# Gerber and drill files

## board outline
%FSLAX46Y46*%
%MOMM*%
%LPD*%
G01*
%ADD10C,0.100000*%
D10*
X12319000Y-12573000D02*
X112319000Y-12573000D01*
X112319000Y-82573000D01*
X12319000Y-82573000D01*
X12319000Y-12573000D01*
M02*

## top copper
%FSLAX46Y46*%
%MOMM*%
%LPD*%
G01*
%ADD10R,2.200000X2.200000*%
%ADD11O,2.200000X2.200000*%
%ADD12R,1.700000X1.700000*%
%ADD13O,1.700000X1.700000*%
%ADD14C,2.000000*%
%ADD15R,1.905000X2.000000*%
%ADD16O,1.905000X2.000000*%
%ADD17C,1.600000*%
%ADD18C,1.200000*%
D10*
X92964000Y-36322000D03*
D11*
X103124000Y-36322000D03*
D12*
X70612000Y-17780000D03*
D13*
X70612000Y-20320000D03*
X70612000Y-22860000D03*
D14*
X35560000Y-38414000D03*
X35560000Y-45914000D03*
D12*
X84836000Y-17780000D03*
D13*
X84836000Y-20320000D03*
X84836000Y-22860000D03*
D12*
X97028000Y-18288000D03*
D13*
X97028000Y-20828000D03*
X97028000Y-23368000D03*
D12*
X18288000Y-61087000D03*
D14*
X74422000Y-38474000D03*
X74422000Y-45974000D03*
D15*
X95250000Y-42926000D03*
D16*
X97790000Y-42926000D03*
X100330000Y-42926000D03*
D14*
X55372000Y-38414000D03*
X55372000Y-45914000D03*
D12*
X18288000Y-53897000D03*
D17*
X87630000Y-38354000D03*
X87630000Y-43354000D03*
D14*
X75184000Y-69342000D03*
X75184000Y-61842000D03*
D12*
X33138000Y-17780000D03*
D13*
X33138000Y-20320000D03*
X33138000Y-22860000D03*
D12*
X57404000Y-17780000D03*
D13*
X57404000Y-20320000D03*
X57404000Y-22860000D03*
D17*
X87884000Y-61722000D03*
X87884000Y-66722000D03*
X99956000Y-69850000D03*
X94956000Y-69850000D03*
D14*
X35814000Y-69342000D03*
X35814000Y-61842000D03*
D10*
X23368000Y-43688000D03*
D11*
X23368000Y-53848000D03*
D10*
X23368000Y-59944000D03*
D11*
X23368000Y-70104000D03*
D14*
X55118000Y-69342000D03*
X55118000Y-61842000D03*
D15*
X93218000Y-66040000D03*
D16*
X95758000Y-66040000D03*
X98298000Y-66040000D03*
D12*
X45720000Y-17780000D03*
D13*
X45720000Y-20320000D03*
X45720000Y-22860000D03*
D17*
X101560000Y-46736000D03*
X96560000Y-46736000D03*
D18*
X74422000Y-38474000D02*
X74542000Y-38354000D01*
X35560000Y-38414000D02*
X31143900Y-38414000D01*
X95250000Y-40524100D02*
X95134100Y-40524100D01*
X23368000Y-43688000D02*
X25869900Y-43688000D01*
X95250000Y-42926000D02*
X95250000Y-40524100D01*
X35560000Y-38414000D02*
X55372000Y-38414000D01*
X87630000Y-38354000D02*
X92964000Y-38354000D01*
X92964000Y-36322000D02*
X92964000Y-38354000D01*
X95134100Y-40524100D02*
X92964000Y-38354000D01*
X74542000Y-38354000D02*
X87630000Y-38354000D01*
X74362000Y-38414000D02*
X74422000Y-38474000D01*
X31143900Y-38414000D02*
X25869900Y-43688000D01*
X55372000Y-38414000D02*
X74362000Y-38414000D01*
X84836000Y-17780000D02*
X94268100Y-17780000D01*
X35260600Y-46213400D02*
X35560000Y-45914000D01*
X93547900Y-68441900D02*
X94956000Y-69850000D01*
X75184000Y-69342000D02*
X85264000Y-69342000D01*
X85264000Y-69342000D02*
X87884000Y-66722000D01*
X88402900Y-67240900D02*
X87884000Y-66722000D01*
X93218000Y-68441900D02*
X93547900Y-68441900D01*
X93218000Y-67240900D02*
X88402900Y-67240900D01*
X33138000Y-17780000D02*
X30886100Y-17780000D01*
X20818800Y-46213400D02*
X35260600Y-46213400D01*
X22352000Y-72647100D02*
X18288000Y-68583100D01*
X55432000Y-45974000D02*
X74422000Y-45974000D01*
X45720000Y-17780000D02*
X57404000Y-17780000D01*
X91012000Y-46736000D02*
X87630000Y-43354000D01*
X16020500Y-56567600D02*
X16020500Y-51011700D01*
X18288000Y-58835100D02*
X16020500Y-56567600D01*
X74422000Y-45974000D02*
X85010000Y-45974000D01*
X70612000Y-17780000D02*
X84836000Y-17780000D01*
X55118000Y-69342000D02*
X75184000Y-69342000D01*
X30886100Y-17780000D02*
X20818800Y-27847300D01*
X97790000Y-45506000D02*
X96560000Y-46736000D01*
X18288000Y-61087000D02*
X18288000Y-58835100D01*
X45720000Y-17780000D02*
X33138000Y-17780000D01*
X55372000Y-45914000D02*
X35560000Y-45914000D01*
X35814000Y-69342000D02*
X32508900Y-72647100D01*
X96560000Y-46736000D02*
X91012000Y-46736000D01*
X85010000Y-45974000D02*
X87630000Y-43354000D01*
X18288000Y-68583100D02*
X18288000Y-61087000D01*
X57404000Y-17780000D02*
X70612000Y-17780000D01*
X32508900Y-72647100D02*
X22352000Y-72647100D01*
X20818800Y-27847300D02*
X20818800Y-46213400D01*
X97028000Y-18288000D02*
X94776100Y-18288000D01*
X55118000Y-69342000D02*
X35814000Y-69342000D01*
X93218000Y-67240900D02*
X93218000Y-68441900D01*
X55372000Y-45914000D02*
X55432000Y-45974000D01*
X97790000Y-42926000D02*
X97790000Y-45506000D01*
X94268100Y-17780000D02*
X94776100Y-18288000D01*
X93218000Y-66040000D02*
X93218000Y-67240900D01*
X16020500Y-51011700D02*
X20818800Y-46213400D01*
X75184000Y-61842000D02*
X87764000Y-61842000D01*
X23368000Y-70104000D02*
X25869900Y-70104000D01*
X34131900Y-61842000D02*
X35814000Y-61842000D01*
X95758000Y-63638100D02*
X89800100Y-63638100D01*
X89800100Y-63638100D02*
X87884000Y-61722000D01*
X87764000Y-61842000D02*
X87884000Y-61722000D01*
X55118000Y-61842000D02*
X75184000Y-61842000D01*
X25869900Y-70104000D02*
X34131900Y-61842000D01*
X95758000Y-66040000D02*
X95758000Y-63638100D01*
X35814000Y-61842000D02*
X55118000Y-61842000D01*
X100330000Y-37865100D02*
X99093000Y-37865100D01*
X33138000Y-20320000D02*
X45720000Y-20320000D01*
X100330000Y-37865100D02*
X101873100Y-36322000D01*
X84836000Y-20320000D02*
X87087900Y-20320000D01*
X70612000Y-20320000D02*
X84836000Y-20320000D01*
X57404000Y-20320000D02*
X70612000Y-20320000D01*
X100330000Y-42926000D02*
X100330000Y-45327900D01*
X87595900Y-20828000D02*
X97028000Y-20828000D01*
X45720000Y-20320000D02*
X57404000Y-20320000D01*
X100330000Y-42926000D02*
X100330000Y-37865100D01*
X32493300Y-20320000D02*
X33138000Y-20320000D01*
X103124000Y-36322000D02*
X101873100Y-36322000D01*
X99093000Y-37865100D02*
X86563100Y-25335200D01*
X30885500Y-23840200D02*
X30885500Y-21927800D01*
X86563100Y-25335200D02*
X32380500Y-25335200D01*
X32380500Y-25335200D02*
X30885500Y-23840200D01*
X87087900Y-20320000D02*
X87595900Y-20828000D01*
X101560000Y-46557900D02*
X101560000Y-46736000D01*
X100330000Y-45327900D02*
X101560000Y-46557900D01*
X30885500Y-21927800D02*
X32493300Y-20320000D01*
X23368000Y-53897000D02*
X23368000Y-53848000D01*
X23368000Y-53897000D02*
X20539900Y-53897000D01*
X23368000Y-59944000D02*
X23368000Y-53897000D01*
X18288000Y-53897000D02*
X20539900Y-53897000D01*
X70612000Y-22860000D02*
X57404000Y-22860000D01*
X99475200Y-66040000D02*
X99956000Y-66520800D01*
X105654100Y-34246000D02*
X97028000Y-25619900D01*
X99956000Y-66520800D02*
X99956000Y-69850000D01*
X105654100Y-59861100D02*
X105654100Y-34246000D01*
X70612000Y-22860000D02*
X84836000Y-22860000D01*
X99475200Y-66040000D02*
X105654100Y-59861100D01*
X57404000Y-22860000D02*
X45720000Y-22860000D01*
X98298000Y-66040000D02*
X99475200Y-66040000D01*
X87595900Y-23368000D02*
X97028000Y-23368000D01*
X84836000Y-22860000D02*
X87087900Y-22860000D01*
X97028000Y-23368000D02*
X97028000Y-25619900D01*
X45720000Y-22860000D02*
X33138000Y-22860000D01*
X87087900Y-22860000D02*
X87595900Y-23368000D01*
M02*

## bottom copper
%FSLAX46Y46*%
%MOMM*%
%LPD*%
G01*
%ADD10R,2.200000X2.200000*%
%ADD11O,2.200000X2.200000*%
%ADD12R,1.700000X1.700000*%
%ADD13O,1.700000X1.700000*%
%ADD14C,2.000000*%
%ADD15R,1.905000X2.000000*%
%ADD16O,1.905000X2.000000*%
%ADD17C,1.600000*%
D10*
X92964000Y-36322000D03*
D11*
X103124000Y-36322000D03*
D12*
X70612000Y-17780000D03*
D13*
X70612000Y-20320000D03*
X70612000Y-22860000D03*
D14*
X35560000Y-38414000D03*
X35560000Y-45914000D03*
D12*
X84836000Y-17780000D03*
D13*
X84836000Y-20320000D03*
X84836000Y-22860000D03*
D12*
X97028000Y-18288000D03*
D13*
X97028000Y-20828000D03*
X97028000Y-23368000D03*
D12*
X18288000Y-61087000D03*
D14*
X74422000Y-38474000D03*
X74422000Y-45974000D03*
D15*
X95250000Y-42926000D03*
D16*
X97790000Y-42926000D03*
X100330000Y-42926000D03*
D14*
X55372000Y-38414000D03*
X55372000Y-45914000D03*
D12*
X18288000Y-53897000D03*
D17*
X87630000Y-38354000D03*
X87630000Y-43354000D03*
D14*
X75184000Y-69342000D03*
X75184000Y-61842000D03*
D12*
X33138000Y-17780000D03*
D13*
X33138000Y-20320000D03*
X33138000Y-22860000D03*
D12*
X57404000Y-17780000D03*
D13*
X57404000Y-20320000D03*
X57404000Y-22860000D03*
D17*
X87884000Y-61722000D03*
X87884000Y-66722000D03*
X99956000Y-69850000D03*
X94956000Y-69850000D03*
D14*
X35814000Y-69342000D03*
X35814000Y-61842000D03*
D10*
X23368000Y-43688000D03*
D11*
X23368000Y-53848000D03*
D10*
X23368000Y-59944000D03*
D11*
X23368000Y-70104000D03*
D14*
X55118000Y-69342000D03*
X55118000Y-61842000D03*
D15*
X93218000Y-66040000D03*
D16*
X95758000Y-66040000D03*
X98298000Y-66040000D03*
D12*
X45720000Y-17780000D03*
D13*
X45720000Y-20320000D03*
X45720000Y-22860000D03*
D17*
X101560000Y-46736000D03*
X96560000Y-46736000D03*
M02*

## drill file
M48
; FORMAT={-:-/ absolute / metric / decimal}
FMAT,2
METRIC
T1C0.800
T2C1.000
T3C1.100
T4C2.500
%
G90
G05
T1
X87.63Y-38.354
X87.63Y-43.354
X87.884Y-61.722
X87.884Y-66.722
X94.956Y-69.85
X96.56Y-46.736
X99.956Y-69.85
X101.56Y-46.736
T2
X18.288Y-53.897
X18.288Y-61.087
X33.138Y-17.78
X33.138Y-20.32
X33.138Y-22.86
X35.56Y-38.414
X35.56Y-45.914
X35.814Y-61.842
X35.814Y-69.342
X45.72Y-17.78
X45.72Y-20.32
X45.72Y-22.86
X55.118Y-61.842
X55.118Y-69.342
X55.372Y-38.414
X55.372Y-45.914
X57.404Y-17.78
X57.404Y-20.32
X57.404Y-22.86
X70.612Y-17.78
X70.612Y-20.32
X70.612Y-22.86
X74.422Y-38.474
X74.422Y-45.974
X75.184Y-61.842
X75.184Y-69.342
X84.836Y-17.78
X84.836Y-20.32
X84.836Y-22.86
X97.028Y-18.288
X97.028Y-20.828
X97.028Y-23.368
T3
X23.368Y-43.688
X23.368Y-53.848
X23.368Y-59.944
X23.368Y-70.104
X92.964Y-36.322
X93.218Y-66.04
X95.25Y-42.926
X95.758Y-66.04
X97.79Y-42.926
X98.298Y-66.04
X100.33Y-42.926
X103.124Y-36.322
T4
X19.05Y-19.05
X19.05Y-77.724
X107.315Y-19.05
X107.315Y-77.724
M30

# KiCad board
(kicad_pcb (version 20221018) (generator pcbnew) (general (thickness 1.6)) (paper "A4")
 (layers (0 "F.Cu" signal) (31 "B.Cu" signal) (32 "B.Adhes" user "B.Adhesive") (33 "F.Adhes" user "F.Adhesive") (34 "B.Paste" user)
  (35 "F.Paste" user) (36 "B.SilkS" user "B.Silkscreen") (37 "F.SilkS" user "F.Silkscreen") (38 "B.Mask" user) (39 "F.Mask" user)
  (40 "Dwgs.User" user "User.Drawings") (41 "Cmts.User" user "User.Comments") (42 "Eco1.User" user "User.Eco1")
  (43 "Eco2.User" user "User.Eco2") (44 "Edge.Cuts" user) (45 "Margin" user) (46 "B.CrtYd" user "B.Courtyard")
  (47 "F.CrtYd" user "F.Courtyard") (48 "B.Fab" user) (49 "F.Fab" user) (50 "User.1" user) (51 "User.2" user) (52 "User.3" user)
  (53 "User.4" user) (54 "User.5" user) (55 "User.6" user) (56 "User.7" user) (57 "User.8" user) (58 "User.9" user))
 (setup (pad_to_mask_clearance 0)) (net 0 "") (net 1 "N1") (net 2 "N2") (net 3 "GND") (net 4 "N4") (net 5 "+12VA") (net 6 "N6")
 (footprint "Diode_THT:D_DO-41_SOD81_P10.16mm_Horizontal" (layer "F.Cu") (at 92.964 36.322)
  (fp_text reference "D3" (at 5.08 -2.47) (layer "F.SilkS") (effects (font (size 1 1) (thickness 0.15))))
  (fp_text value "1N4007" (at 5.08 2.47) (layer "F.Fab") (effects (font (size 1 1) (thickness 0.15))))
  (pad "1" thru_hole rect (at 0 0) (size 2.2 2.2) (drill 1.1) (layers "*.Cu" "*.Mask") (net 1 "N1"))
  (pad "2" thru_hole oval (at 10.16 0) (size 2.2 2.2) (drill 1.1) (layers "*.Cu" "*.Mask") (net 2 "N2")))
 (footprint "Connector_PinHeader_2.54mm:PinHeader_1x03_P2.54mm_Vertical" (layer "F.Cu") (at 70.612 17.78)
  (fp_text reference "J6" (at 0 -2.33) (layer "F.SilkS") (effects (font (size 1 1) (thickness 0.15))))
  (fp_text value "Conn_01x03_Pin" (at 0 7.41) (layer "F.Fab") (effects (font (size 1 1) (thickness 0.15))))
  (pad "1" thru_hole rect (at 0 0) (size 1.7 1.7) (drill 1) (layers "*.Cu" "*.Mask") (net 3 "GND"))
  (pad "2" thru_hole oval (at 0 2.54) (size 1.7 1.7) (drill 1) (layers "*.Cu" "*.Mask") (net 2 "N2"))
  (pad "3" thru_hole oval (at 0 5.08) (size 1.7 1.7) (drill 1) (layers "*.Cu" "*.Mask") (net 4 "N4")))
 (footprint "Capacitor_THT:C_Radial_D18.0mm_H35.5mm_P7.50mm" (layer "F.Cu") (at 35.56 38.414 -90)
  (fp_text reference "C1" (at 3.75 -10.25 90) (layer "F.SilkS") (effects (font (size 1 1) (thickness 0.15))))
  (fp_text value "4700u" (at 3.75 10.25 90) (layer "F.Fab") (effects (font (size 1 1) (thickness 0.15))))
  (pad "1" thru_hole circle (at 0 0 270) (size 2 2) (drill 1) (layers "*.Cu" "*.Mask") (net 1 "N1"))
  (pad "2" thru_hole circle (at 7.5 0 270) (size 2 2) (drill 1) (layers "*.Cu" "*.Mask") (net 3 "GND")))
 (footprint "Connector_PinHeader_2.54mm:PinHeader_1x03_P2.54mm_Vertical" (layer "F.Cu") (at 84.836 17.78)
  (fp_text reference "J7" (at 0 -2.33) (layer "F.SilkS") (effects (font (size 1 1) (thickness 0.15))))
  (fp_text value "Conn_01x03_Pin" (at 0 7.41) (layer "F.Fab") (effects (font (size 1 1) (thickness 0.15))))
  (pad "1" thru_hole rect (at 0 0) (size 1.7 1.7) (drill 1) (layers "*.Cu" "*.Mask") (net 3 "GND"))
  (pad "2" thru_hole oval (at 0 2.54) (size 1.7 1.7) (drill 1) (layers "*.Cu" "*.Mask") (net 2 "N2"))
  (pad "3" thru_hole oval (at 0 5.08) (size 1.7 1.7) (drill 1) (layers "*.Cu" "*.Mask") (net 4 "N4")))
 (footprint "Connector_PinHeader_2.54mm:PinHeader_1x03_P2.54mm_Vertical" (layer "F.Cu") (at 97.028 18.288)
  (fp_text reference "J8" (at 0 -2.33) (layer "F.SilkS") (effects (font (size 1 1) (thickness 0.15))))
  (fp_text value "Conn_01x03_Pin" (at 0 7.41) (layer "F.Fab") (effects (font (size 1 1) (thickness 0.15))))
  (pad "1" thru_hole rect (at 0 0) (size 1.7 1.7) (drill 1) (layers "*.Cu" "*.Mask") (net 3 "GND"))
  (pad "2" thru_hole oval (at 0 2.54) (size 1.7 1.7) (drill 1) (layers "*.Cu" "*.Mask") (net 2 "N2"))
  (pad "3" thru_hole oval (at 0 5.08) (size 1.7 1.7) (drill 1) (layers "*.Cu" "*.Mask") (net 4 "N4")))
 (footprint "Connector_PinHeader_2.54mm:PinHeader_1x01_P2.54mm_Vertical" (layer "F.Cu") (at 18.288 61.087)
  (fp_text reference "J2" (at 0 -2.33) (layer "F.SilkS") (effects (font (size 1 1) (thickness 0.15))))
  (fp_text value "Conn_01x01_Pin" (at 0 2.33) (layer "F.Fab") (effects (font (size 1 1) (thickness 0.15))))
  (pad "1" thru_hole rect (at 0 0) (size 1.7 1.7) (drill 1) (layers "*.Cu" "*.Mask") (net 3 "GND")))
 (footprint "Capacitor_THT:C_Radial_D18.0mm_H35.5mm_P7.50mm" (layer "F.Cu") (at 74.422 38.474 -90)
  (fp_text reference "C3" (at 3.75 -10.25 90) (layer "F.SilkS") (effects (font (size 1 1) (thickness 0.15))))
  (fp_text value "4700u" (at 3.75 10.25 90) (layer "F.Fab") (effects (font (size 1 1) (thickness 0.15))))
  (pad "1" thru_hole circle (at 0 0 270) (size 2 2) (drill 1) (layers "*.Cu" "*.Mask") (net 1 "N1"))
  (pad "2" thru_hole circle (at 7.5 0 270) (size 2 2) (drill 1) (layers "*.Cu" "*.Mask") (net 3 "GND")))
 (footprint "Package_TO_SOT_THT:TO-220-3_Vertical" (layer "F.Cu") (at 95.25 42.926)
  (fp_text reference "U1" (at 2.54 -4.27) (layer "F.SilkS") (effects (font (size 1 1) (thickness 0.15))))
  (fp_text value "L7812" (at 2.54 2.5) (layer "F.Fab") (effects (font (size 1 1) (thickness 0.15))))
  (pad "1" thru_hole rect (at 0 0) (size 1.905 2) (drill 1.1) (layers "*.Cu" "*.Mask") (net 1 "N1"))
  (pad "2" thru_hole oval (at 2.54 0) (size 1.905 2) (drill 1.1) (layers "*.Cu" "*.Mask") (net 3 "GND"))
  (pad "3" thru_hole oval (at 5.08 0) (size 1.905 2) (drill 1.1) (layers "*.Cu" "*.Mask") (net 2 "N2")))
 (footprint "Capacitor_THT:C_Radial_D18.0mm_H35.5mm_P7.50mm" (layer "F.Cu") (at 55.372 38.414 -90)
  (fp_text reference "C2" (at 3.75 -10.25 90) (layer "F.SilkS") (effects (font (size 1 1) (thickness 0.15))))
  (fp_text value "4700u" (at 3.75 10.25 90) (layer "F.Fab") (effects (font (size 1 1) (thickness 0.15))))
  (pad "1" thru_hole circle (at 0 0 270) (size 2 2) (drill 1) (layers "*.Cu" "*.Mask") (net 1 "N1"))
  (pad "2" thru_hole circle (at 7.5 0 270) (size 2 2) (drill 1) (layers "*.Cu" "*.Mask") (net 3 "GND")))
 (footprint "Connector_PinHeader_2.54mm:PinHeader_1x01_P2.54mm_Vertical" (layer "F.Cu") (at 18.288 53.897)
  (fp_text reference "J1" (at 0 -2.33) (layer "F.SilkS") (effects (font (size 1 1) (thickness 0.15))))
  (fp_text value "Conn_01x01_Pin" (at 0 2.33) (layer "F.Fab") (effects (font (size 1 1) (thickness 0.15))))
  (pad "1" thru_hole rect (at 0 0) (size 1.7 1.7) (drill 1) (layers "*.Cu" "*.Mask") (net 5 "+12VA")))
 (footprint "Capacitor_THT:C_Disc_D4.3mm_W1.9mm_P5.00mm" (layer "F.Cu") (at 87.63 38.354 -90)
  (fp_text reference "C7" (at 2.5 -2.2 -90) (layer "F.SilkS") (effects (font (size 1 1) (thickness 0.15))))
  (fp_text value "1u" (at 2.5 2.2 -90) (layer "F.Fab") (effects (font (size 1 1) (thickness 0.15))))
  (pad "1" thru_hole circle (at 0 0 270) (size 1.6 1.6) (drill 0.8) (layers "*.Cu" "*.Mask") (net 1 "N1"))
  (pad "2" thru_hole circle (at 5 0 270) (size 1.6 1.6) (drill 0.8) (layers "*.Cu" "*.Mask") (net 3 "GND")))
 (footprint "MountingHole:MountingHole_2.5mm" (layer "F.Cu") (at 19.05 19.05)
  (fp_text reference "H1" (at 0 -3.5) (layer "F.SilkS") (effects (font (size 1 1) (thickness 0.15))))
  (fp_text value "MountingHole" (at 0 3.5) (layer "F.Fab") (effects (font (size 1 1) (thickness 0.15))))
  (pad "" np_thru_hole circle (at 0 0) (size 2.5 2.5) (drill 2.5) (layers "*.Cu" "*.Mask")))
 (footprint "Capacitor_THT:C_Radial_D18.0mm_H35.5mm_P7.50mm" (layer "F.Cu") (at 75.184 69.342 90)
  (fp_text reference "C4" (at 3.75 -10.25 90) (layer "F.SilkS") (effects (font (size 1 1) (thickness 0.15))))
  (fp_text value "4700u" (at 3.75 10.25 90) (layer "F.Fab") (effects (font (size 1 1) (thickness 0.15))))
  (pad "1" thru_hole circle (at 0 0 90) (size 2 2) (drill 1) (layers "*.Cu" "*.Mask") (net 3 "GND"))
  (pad "2" thru_hole circle (at 7.5 0 90) (size 2 2) (drill 1) (layers "*.Cu" "*.Mask") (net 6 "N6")))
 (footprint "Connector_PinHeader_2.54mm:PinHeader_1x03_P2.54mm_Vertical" (layer "F.Cu") (at 33.138 17.78)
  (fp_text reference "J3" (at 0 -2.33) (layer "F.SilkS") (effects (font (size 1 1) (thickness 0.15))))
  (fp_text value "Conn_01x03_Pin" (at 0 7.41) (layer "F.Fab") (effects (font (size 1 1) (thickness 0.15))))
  (pad "1" thru_hole rect (at 0 0) (size 1.7 1.7) (drill 1) (layers "*.Cu" "*.Mask") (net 3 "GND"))
  (pad "2" thru_hole oval (at 0 2.54) (size 1.7 1.7) (drill 1) (layers "*.Cu" "*.Mask") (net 2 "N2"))
  (pad "3" thru_hole oval (at 0 5.08) (size 1.7 1.7) (drill 1) (layers "*.Cu" "*.Mask") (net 4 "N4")))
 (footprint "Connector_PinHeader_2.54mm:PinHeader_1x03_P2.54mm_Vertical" (layer "F.Cu") (at 57.404 17.78)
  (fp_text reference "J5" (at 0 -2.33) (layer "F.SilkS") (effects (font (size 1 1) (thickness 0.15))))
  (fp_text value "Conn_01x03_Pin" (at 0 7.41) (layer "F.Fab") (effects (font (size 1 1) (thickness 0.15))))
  (pad "1" thru_hole rect (at 0 0) (size 1.7 1.7) (drill 1) (layers "*.Cu" "*.Mask") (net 3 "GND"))
  (pad "2" thru_hole oval (at 0 2.54) (size 1.7 1.7) (drill 1) (layers "*.Cu" "*.Mask") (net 2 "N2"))
  (pad "3" thru_hole oval (at 0 5.08) (size 1.7 1.7) (drill 1) (layers "*.Cu" "*.Mask") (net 4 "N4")))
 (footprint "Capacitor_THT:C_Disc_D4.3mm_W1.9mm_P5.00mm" (layer "F.Cu") (at 87.884 61.722 -90)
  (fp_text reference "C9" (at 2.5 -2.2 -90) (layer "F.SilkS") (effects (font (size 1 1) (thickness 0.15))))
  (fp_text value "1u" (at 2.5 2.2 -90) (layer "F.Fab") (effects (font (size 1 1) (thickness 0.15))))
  (pad "1" thru_hole circle (at 0 0 270) (size 1.6 1.6) (drill 0.8) (layers "*.Cu" "*.Mask") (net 6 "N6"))
  (pad "2" thru_hole circle (at 5 0 270) (size 1.6 1.6) (drill 0.8) (layers "*.Cu" "*.Mask") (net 3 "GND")))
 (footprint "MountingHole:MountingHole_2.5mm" (layer "F.Cu") (at 19.05 77.724)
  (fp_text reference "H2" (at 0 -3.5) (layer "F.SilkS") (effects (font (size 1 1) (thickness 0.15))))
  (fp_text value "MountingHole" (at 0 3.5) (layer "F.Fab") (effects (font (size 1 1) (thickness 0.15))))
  (pad "" np_thru_hole circle (at 0 0) (size 2.5 2.5) (drill 2.5) (layers "*.Cu" "*.Mask")))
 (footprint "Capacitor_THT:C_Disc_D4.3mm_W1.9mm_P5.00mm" (layer "F.Cu") (at 99.956 69.85 180)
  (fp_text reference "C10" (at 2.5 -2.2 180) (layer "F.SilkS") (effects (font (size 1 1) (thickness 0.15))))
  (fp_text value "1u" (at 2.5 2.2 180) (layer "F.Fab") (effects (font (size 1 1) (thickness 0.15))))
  (pad "1" thru_hole circle (at 0 0 180) (size 1.6 1.6) (drill 0.8) (layers "*.Cu" "*.Mask") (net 4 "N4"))
  (pad "2" thru_hole circle (at 5 0 180) (size 1.6 1.6) (drill 0.8) (layers "*.Cu" "*.Mask") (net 3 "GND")))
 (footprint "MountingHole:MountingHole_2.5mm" (layer "F.Cu") (at 107.315 77.724)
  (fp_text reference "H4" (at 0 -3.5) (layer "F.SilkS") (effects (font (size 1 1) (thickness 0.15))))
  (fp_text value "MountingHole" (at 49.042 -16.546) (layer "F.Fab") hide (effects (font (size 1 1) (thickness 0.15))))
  (pad "" np_thru_hole circle (at 0 0) (size 2.5 2.5) (drill 2.5) (layers "*.Cu" "*.Mask")))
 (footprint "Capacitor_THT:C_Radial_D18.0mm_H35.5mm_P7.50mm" (layer "F.Cu") (at 35.814 69.342 90)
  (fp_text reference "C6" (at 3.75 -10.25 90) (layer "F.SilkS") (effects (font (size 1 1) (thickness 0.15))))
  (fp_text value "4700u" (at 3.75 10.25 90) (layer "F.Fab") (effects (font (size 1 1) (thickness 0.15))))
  (pad "1" thru_hole circle (at 0 0 90) (size 2 2) (drill 1) (layers "*.Cu" "*.Mask") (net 3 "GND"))
  (pad "2" thru_hole circle (at 7.5 0 90) (size 2 2) (drill 1) (layers "*.Cu" "*.Mask") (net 6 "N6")))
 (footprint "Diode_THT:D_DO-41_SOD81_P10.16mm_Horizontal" (layer "F.Cu") (at 23.368 43.688 -90)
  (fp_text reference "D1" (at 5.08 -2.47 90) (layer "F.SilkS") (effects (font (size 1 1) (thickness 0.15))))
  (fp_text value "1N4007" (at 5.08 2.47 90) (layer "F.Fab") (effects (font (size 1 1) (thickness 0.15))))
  (pad "1" thru_hole rect (at 0 0 270) (size 2.2 2.2) (drill 1.1) (layers "*.Cu" "*.Mask") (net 1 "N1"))
  (pad "2" thru_hole oval (at 10.16 0 270) (size 2.2 2.2) (drill 1.1) (layers "*.Cu" "*.Mask") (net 5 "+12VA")))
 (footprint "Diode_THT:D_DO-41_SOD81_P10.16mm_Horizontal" (layer "F.Cu") (at 23.368 59.944 -90)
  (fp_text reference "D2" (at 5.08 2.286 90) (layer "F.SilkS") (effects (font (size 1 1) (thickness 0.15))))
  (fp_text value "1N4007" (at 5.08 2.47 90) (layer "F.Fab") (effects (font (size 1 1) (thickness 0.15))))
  (pad "1" thru_hole rect (at 0 0 270) (size 2.2 2.2) (drill 1.1) (layers "*.Cu" "*.Mask") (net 5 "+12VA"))
  (pad "2" thru_hole oval (at 10.16 0 270) (size 2.2 2.2) (drill 1.1) (layers "*.Cu" "*.Mask") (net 6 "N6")))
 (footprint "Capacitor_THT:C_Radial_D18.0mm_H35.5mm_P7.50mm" (layer "F.Cu") (at 55.118 69.342 90)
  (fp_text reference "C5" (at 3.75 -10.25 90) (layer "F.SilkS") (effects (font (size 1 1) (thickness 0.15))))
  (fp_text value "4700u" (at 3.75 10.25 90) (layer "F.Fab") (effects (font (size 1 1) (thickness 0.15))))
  (pad "1" thru_hole circle (at 0 0 90) (size 2 2) (drill 1) (layers "*.Cu" "*.Mask") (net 3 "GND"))
  (pad "2" thru_hole circle (at 7.5 0 90) (size 2 2) (drill 1) (layers "*.Cu" "*.Mask") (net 6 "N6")))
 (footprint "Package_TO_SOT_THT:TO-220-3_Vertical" (layer "F.Cu") (at 93.218 66.04)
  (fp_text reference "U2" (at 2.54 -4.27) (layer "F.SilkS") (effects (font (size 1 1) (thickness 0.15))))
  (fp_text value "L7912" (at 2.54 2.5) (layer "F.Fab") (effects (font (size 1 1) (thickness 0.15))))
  (pad "1" thru_hole rect (at 0 0) (size 1.905 2) (drill 1.1) (layers "*.Cu" "*.Mask") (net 3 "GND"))
  (pad "2" thru_hole oval (at 2.54 0) (size 1.905 2) (drill 1.1) (layers "*.Cu" "*.Mask") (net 6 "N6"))
  (pad "3" thru_hole oval (at 5.08 0) (size 1.905 2) (drill 1.1) (layers "*.Cu" "*.Mask") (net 4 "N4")))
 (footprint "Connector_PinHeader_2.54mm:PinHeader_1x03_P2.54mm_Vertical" (layer "F.Cu") (at 45.72 17.78)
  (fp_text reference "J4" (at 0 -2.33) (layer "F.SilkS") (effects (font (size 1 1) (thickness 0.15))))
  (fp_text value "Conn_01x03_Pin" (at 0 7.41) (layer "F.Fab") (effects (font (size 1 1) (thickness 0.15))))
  (pad "1" thru_hole rect (at 0 0) (size 1.7 1.7) (drill 1) (layers "*.Cu" "*.Mask") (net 3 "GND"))
  (pad "2" thru_hole oval (at 0 2.54) (size 1.7 1.7) (drill 1) (layers "*.Cu" "*.Mask") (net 2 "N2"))
  (pad "3" thru_hole oval (at 0 5.08) (size 1.7 1.7) (drill 1) (layers "*.Cu" "*.Mask") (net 4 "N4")))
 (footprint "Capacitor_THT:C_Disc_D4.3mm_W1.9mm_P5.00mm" (layer "F.Cu") (at 101.56 46.736 180)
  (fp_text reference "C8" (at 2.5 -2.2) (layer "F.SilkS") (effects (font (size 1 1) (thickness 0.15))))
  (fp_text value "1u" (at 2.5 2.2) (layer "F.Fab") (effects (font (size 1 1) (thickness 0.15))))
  (pad "1" thru_hole circle (at 0 0 180) (size 1.6 1.6) (drill 0.8) (layers "*.Cu" "*.Mask") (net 2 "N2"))
  (pad "2" thru_hole circle (at 5 0 180) (size 1.6 1.6) (drill 0.8) (layers "*.Cu" "*.Mask") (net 3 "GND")))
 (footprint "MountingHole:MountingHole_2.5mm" (layer "F.Cu") (at 107.315 19.05)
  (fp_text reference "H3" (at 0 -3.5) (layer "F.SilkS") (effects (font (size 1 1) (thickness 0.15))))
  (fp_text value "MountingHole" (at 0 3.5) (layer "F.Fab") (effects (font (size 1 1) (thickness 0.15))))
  (pad "" np_thru_hole circle (at 0 0) (size 2.5 2.5) (drill 2.5) (layers "*.Cu" "*.Mask")))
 (gr_rect (start 12.319 12.573) (end 112.319 82.573) (stroke (width 0.1) (type default)) (fill none) (layer "Edge.Cuts"))
 (segment (start 74.422 38.474) (end 74.542 38.354) (width 1.2) (layer "F.Cu") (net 1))
 (segment (start 35.56 38.414) (end 31.1439 38.414) (width 1.2) (layer "F.Cu") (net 1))
 (segment (start 95.25 40.5241) (end 95.1341 40.5241) (width 1.2) (layer "F.Cu") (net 1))
 (segment (start 23.368 43.688) (end 25.8699 43.688) (width 1.2) (layer "F.Cu") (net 1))
 (segment (start 95.25 42.926) (end 95.25 40.5241) (width 1.2) (layer "F.Cu") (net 1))
 (segment (start 35.56 38.414) (end 55.372 38.414) (width 1.2) (layer "F.Cu") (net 1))
 (segment (start 87.63 38.354) (end 92.964 38.354) (width 1.2) (layer "F.Cu") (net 1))
 (segment (start 92.964 36.322) (end 92.964 38.354) (width 1.2) (layer "F.Cu") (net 1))
 (segment (start 95.1341 40.5241) (end 92.964 38.354) (width 1.2) (layer "F.Cu") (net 1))
 (segment (start 74.542 38.354) (end 87.63 38.354) (width 1.2) (layer "F.Cu") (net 1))
 (segment (start 74.362 38.414) (end 74.422 38.474) (width 1.2) (layer "F.Cu") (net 1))
 (segment (start 31.1439 38.414) (end 25.8699 43.688) (width 1.2) (layer "F.Cu") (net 1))
 (segment (start 55.372 38.414) (end 74.362 38.414) (width 1.2) (layer "F.Cu") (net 1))
 (segment (start 84.836 17.78) (end 94.2681 17.78) (width 1.2) (layer "F.Cu") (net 3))
 (segment (start 35.2606 46.2134) (end 35.56 45.914) (width 1.2) (layer "F.Cu") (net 3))
 (segment (start 93.5479 68.4419) (end 94.956 69.85) (width 1.2) (layer "F.Cu") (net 3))
 (segment (start 75.184 69.342) (end 85.264 69.342) (width 1.2) (layer "F.Cu") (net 3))
 (segment (start 85.264 69.342) (end 87.884 66.722) (width 1.2) (layer "F.Cu") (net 3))
 (segment (start 88.4029 67.2409) (end 87.884 66.722) (width 1.2) (layer "F.Cu") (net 3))
 (segment (start 93.218 68.4419) (end 93.5479 68.4419) (width 1.2) (layer "F.Cu") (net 3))
 (segment (start 93.218 67.2409) (end 88.4029 67.2409) (width 1.2) (layer "F.Cu") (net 3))
 (segment (start 33.138 17.78) (end 30.8861 17.78) (width 1.2) (layer "F.Cu") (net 3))
 (segment (start 20.8188 46.2134) (end 35.2606 46.2134) (width 1.2) (layer "F.Cu") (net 3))
 (segment (start 22.352 72.6471) (end 18.288 68.5831) (width 1.2) (layer "F.Cu") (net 3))
 (segment (start 55.432 45.974) (end 74.422 45.974) (width 1.2) (layer "F.Cu") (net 3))
 (segment (start 45.72 17.78) (end 57.404 17.78) (width 1.2) (layer "F.Cu") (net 3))
 (segment (start 91.012 46.736) (end 87.63 43.354) (width 1.2) (layer "F.Cu") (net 3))
 (segment (start 16.0205 56.5676) (end 16.0205 51.0117) (width 1.2) (layer "F.Cu") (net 3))
 (segment (start 18.288 58.8351) (end 16.0205 56.5676) (width 1.2) (layer "F.Cu") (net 3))
 (segment (start 74.422 45.974) (end 85.01 45.974) (width 1.2) (layer "F.Cu") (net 3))
 (segment (start 70.612 17.78) (end 84.836 17.78) (width 1.2) (layer "F.Cu") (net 3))
 (segment (start 55.118 69.342) (end 75.184 69.342) (width 1.2) (layer "F.Cu") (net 3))
 (segment (start 30.8861 17.78) (end 20.8188 27.8473) (width 1.2) (layer "F.Cu") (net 3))
 (segment (start 97.79 45.506) (end 96.56 46.736) (width 1.2) (layer "F.Cu") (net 3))
 (segment (start 18.288 61.087) (end 18.288 58.8351) (width 1.2) (layer "F.Cu") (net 3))
 (segment (start 45.72 17.78) (end 33.138 17.78) (width 1.2) (layer "F.Cu") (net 3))
 (segment (start 55.372 45.914) (end 35.56 45.914) (width 1.2) (layer "F.Cu") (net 3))
 (segment (start 35.814 69.342) (end 32.5089 72.6471) (width 1.2) (layer "F.Cu") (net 3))
 (segment (start 96.56 46.736) (end 91.012 46.736) (width 1.2) (layer "F.Cu") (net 3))
 (segment (start 85.01 45.974) (end 87.63 43.354) (width 1.2) (layer "F.Cu") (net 3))
 (segment (start 18.288 68.5831) (end 18.288 61.087) (width 1.2) (layer "F.Cu") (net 3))
 (segment (start 57.404 17.78) (end 70.612 17.78) (width 1.2) (layer "F.Cu") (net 3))
 (segment (start 32.5089 72.6471) (end 22.352 72.6471) (width 1.2) (layer "F.Cu") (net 3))
 (segment (start 20.8188 27.8473) (end 20.8188 46.2134) (width 1.2) (layer "F.Cu") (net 3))
 (segment (start 97.028 18.288) (end 94.7761 18.288) (width 1.2) (layer "F.Cu") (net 3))
 (segment (start 55.118 69.342) (end 35.814 69.342) (width 1.2) (layer "F.Cu") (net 3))
 (segment (start 93.218 67.2409) (end 93.218 68.4419) (width 1.2) (layer "F.Cu") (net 3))
 (segment (start 55.372 45.914) (end 55.432 45.974) (width 1.2) (layer "F.Cu") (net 3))
 (segment (start 97.79 42.926) (end 97.79 45.506) (width 1.2) (layer "F.Cu") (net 3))
 (segment (start 94.2681 17.78) (end 94.7761 18.288) (width 1.2) (layer "F.Cu") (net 3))
 (segment (start 93.218 66.04) (end 93.218 67.2409) (width 1.2) (layer "F.Cu") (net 3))
 (segment (start 16.0205 51.0117) (end 20.8188 46.2134) (width 1.2) (layer "F.Cu") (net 3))
 (segment (start 75.184 61.842) (end 87.764 61.842) (width 1.2) (layer "F.Cu") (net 6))
 (segment (start 23.368 70.104) (end 25.8699 70.104) (width 1.2) (layer "F.Cu") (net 6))
 (segment (start 34.1319 61.842) (end 35.814 61.842) (width 1.2) (layer "F.Cu") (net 6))
 (segment (start 95.758 63.6381) (end 89.8001 63.6381) (width 1.2) (layer "F.Cu") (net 6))
 (segment (start 89.8001 63.6381) (end 87.884 61.722) (width 1.2) (layer "F.Cu") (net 6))
 (segment (start 87.764 61.842) (end 87.884 61.722) (width 1.2) (layer "F.Cu") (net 6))
 (segment (start 55.118 61.842) (end 75.184 61.842) (width 1.2) (layer "F.Cu") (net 6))
 (segment (start 25.8699 70.104) (end 34.1319 61.842) (width 1.2) (layer "F.Cu") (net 6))
 (segment (start 95.758 66.04) (end 95.758 63.6381) (width 1.2) (layer "F.Cu") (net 6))
 (segment (start 35.814 61.842) (end 55.118 61.842) (width 1.2) (layer "F.Cu") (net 6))
 (segment (start 100.33 37.8651) (end 99.093 37.8651) (width 1.2) (layer "F.Cu") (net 2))
 (segment (start 33.138 20.32) (end 45.72 20.32) (width 1.2) (layer "F.Cu") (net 2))
 (segment (start 100.33 37.8651) (end 101.8731 36.322) (width 1.2) (layer "F.Cu") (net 2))
 (segment (start 84.836 20.32) (end 87.0879 20.32) (width 1.2) (layer "F.Cu") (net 2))
 (segment (start 70.612 20.32) (end 84.836 20.32) (width 1.2) (layer "F.Cu") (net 2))
 (segment (start 57.404 20.32) (end 70.612 20.32) (width 1.2) (layer "F.Cu") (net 2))
 (segment (start 100.33 42.926) (end 100.33 45.3279) (width 1.2) (layer "F.Cu") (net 2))
 (segment (start 87.5959 20.828) (end 97.028 20.828) (width 1.2) (layer "F.Cu") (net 2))
 (segment (start 45.72 20.32) (end 57.404 20.32) (width 1.2) (layer "F.Cu") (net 2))
 (segment (start 100.33 42.926) (end 100.33 37.8651) (width 1.2) (layer "F.Cu") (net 2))
 (segment (start 32.4933 20.32) (end 33.138 20.32) (width 1.2) (layer "F.Cu") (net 2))
 (segment (start 103.124 36.322) (end 101.8731 36.322) (width 1.2) (layer "F.Cu") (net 2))
 (segment (start 99.093 37.8651) (end 86.5631 25.3352) (width 1.2) (layer "F.Cu") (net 2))
 (segment (start 30.8855 23.8402) (end 30.8855 21.9278) (width 1.2) (layer "F.Cu") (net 2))
 (segment (start 86.5631 25.3352) (end 32.3805 25.3352) (width 1.2) (layer "F.Cu") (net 2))
 (segment (start 32.3805 25.3352) (end 30.8855 23.8402) (width 1.2) (layer "F.Cu") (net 2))
 (segment (start 87.0879 20.32) (end 87.5959 20.828) (width 1.2) (layer "F.Cu") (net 2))
 (segment (start 101.56 46.5579) (end 101.56 46.736) (width 1.2) (layer "F.Cu") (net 2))
 (segment (start 100.33 45.3279) (end 101.56 46.5579) (width 1.2) (layer "F.Cu") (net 2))
 (segment (start 30.8855 21.9278) (end 32.4933 20.32) (width 1.2) (layer "F.Cu") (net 2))
 (segment (start 23.368 53.897) (end 23.368 53.848) (width 1.2) (layer "F.Cu") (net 5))
 (segment (start 23.368 53.897) (end 20.5399 53.897) (width 1.2) (layer "F.Cu") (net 5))
 (segment (start 23.368 59.944) (end 23.368 53.897) (width 1.2) (layer "F.Cu") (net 5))
 (segment (start 18.288 53.897) (end 20.5399 53.897) (width 1.2) (layer "F.Cu") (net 5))
 (segment (start 70.612 22.86) (end 57.404 22.86) (width 1.2) (layer "F.Cu") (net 4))
 (segment (start 99.4752 66.04) (end 99.956 66.5208) (width 1.2) (layer "F.Cu") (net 4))
 (segment (start 105.6541 34.246) (end 97.028 25.6199) (width 1.2) (layer "F.Cu") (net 4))
 (segment (start 99.956 66.5208) (end 99.956 69.85) (width 1.2) (layer "F.Cu") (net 4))
 (segment (start 105.6541 59.8611) (end 105.6541 34.246) (width 1.2) (layer "F.Cu") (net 4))
 (segment (start 70.612 22.86) (end 84.836 22.86) (width 1.2) (layer "F.Cu") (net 4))
 (segment (start 99.4752 66.04) (end 105.6541 59.8611) (width 1.2) (layer "F.Cu") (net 4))
 (segment (start 57.404 22.86) (end 45.72 22.86) (width 1.2) (layer "F.Cu") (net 4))
 (segment (start 98.298 66.04) (end 99.4752 66.04) (width 1.2) (layer "F.Cu") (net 4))
 (segment (start 87.5959 23.368) (end 97.028 23.368) (width 1.2) (layer "F.Cu") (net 4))
 (segment (start 84.836 22.86) (end 87.0879 22.86) (width 1.2) (layer "F.Cu") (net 4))
 (segment (start 97.028 23.368) (end 97.028 25.6199) (width 1.2) (layer "F.Cu") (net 4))
 (segment (start 45.72 22.86) (end 33.138 22.86) (width 1.2) (layer "F.Cu") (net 4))
 (segment (start 87.0879 22.86) (end 87.5959 23.368) (width 1.2) (layer "F.Cu") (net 4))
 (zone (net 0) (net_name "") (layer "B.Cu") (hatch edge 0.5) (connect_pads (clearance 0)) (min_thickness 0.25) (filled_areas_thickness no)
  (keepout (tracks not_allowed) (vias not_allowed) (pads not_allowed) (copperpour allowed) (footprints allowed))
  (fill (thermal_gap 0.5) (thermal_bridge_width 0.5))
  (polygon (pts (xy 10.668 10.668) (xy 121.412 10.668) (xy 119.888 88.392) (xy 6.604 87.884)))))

